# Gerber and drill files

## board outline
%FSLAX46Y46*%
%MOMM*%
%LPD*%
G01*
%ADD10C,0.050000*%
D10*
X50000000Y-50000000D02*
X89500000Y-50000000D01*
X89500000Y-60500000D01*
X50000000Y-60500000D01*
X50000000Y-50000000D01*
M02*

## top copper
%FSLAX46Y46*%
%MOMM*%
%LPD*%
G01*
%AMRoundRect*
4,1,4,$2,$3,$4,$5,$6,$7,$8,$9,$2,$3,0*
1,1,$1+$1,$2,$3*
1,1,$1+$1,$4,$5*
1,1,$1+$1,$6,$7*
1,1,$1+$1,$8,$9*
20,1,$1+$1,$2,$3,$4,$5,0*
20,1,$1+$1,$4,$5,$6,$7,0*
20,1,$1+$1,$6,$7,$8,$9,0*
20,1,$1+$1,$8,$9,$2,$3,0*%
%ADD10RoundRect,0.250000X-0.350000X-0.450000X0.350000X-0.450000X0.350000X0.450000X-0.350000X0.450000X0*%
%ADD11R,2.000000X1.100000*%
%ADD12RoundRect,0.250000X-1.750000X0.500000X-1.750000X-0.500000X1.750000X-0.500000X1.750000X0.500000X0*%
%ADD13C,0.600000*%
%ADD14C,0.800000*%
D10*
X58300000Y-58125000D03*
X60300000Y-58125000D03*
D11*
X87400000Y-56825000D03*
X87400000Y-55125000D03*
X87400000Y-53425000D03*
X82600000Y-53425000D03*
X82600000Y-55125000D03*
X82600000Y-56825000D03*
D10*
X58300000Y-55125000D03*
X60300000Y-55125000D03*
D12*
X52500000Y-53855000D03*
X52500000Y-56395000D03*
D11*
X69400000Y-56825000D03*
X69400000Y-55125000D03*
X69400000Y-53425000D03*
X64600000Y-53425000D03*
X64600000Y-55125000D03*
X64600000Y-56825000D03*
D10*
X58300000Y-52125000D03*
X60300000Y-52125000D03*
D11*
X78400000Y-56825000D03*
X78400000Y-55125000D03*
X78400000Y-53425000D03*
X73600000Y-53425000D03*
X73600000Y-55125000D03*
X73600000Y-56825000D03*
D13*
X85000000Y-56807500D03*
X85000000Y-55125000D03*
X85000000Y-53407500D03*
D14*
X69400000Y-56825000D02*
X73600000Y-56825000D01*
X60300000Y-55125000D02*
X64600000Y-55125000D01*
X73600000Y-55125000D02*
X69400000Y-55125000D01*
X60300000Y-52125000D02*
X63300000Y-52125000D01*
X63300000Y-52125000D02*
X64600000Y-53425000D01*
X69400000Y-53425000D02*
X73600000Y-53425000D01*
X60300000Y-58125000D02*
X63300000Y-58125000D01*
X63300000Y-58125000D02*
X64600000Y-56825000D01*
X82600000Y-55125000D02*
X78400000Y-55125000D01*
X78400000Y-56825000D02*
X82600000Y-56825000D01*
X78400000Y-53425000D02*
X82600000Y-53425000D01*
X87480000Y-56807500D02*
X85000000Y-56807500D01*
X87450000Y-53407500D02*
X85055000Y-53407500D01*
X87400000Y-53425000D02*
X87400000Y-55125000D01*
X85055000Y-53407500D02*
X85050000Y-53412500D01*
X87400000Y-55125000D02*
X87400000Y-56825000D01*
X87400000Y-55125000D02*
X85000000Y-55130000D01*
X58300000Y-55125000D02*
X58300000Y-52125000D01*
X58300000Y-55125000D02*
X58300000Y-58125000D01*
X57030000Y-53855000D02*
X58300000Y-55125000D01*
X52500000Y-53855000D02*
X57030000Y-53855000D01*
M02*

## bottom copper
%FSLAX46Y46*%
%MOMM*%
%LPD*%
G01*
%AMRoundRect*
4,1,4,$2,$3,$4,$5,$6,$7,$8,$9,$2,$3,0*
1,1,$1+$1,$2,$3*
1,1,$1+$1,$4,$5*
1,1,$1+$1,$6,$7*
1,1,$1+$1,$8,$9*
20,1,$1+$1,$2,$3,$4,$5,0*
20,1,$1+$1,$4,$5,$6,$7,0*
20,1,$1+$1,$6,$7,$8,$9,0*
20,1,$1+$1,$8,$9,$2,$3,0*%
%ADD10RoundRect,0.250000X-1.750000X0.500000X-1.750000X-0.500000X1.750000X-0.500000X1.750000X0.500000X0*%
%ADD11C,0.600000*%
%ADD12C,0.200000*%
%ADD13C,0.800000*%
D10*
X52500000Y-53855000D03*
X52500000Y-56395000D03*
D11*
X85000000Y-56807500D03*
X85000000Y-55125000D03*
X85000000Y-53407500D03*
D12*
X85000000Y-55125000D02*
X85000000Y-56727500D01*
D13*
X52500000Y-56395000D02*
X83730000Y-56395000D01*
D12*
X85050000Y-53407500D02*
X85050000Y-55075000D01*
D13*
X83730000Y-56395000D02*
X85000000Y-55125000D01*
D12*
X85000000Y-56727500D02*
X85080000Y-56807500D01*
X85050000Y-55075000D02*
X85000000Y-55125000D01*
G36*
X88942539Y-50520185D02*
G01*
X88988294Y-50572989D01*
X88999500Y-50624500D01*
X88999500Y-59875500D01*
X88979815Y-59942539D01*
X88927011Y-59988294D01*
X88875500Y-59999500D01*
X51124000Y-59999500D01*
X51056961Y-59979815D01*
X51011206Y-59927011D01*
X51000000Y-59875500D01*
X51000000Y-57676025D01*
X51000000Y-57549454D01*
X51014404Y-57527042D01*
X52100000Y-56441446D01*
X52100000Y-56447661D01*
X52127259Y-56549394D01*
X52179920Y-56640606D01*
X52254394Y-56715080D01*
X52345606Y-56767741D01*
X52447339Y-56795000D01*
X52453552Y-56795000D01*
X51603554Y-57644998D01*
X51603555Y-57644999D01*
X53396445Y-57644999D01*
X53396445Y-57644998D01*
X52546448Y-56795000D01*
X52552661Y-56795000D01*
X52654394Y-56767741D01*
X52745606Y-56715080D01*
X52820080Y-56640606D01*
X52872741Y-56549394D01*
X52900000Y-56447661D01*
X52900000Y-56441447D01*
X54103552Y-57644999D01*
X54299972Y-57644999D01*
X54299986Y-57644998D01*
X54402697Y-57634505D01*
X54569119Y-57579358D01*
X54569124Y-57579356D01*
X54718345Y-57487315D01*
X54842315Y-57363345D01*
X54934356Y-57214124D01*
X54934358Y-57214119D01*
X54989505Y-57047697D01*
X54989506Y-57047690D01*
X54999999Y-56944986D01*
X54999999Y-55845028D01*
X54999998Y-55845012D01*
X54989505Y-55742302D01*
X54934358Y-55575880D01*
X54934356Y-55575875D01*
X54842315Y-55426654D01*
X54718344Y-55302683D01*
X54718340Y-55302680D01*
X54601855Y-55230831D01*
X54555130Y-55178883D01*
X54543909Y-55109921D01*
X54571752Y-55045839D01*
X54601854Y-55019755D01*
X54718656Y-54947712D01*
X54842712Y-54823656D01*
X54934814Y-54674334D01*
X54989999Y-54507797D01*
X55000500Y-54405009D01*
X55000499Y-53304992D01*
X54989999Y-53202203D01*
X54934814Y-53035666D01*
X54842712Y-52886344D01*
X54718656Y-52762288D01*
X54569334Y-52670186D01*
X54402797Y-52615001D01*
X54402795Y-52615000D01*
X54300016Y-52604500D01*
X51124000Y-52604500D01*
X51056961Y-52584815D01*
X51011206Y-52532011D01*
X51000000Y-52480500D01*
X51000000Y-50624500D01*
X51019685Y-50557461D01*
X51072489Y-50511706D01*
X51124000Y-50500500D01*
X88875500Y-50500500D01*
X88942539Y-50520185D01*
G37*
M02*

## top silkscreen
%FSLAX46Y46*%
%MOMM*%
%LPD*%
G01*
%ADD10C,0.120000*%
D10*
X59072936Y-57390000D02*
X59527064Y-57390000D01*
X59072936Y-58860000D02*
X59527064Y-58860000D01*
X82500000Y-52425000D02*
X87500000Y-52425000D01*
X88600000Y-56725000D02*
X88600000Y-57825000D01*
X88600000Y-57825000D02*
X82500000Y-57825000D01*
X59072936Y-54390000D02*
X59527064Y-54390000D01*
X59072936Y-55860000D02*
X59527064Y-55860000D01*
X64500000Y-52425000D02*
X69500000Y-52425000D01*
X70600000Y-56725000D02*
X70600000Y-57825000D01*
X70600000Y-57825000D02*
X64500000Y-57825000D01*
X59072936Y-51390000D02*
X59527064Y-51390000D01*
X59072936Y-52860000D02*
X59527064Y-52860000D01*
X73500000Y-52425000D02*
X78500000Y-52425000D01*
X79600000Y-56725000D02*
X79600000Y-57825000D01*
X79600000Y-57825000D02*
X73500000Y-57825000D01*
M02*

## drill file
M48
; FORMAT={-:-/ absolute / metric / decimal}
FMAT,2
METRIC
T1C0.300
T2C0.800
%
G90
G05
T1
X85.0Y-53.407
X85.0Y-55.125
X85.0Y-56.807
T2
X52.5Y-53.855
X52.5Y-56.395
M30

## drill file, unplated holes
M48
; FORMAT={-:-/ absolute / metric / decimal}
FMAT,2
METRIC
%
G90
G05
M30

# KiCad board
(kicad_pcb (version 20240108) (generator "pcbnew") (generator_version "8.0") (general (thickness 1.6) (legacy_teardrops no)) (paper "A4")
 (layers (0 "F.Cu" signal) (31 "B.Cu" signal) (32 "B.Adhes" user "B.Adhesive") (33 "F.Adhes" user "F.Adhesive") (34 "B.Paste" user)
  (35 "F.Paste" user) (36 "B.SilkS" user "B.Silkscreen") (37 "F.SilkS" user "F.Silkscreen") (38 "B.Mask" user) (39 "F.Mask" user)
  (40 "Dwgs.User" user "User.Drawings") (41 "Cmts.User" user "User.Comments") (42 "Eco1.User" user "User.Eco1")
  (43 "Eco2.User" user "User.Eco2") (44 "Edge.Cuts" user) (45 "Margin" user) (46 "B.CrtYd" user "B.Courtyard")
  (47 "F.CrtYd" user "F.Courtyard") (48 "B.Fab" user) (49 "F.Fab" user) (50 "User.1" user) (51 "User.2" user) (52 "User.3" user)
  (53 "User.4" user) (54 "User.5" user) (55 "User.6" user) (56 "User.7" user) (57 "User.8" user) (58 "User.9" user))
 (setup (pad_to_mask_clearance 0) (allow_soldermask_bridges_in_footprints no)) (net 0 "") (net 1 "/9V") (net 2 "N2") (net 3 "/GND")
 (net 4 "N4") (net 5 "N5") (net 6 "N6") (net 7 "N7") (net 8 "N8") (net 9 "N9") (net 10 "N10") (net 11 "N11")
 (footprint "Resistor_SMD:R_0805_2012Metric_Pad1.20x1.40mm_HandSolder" (layer "F.Cu") (at 59.3 58.125)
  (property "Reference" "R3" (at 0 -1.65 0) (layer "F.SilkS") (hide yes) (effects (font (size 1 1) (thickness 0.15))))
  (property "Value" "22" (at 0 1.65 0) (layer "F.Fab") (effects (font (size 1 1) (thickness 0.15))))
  (fp_line (start -0.227064 -0.735) (end 0.227064 -0.735) (stroke (width 0.12) (type solid)) (layer "F.SilkS"))
  (fp_line (start -0.227064 0.735) (end 0.227064 0.735) (stroke (width 0.12) (type solid)) (layer "F.SilkS"))
  (pad "1" smd roundrect (at -1 0) (size 1.2 1.4) (layers "F.Cu" "F.Paste" "F.Mask") (roundrect_rratio 0.208333) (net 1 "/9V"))
  (pad "2" smd roundrect (at 1 0) (size 1.2 1.4) (layers "F.Cu" "F.Paste" "F.Mask") (roundrect_rratio 0.208333) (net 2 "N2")))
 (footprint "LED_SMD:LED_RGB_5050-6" (layer "F.Cu") (at 85 55.125 180)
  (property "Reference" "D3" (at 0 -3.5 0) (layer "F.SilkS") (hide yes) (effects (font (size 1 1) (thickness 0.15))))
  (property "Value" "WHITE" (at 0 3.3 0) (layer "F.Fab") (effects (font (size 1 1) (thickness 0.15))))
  (fp_line (start 2.5 2.7) (end -2.5 2.7) (stroke (width 0.12) (type solid)) (layer "F.SilkS"))
  (fp_line (start -3.6 -1.6) (end -3.6 -2.7) (stroke (width 0.12) (type solid)) (layer "F.SilkS"))
  (fp_line (start -3.6 -2.7) (end 2.5 -2.7) (stroke (width 0.12) (type solid)) (layer "F.SilkS"))
  (pad "1" smd rect (at -2.4 -1.7 270) (size 1.1 2) (layers "F.Cu" "F.Paste" "F.Mask") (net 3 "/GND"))
  (pad "2" smd rect (at -2.4 0 270) (size 1.1 2) (layers "F.Cu" "F.Paste" "F.Mask") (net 3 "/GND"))
  (pad "3" smd rect (at -2.4 1.7 270) (size 1.1 2) (layers "F.Cu" "F.Paste" "F.Mask") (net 3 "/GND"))
  (pad "4" smd rect (at 2.4 1.7 270) (size 1.1 2) (layers "F.Cu" "F.Paste" "F.Mask") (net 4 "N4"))
  (pad "5" smd rect (at 2.4 0 270) (size 1.1 2) (layers "F.Cu" "F.Paste" "F.Mask") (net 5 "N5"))
  (pad "6" smd rect (at 2.4 -1.7 270) (size 1.1 2) (layers "F.Cu" "F.Paste" "F.Mask") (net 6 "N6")))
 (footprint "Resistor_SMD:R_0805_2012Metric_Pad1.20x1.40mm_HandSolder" (layer "F.Cu") (at 59.3 55.125)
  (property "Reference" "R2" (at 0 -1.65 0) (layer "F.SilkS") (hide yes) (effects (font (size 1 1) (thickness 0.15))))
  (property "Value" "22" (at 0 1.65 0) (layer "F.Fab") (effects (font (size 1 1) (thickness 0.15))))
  (fp_line (start -0.227064 -0.735) (end 0.227064 -0.735) (stroke (width 0.12) (type solid)) (layer "F.SilkS"))
  (fp_line (start -0.227064 0.735) (end 0.227064 0.735) (stroke (width 0.12) (type solid)) (layer "F.SilkS"))
  (pad "1" smd roundrect (at -1 0) (size 1.2 1.4) (layers "F.Cu" "F.Paste" "F.Mask") (roundrect_rratio 0.208333) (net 1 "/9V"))
  (pad "2" smd roundrect (at 1 0) (size 1.2 1.4) (layers "F.Cu" "F.Paste" "F.Mask") (roundrect_rratio 0.208333) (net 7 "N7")))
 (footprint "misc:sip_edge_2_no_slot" (layer "F.Cu") (at 50.5 55.125 -90)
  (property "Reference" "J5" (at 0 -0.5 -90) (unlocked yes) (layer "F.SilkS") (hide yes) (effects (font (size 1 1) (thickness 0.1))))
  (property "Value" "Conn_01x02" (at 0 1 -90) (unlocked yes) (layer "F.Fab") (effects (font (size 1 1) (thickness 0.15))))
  (pad "1" thru_hole roundrect (at -1.27 -2 270) (size 1.5 4) (drill 0.8) (layers "*.Cu" "*.Mask") (remove_unused_layers no)
   (roundrect_rratio 0.1666666667) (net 1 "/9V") (thermal_bridge_angle 45))
  (pad "2" thru_hole roundrect (at 1.27 -2 270) (size 1.5 4) (drill 0.8) (layers "*.Cu" "*.Mask") (remove_unused_layers no)
   (roundrect_rratio 0.1666666667) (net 3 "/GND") (thermal_bridge_angle 45)))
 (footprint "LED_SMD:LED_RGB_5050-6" (layer "F.Cu") (at 67 55.125 180)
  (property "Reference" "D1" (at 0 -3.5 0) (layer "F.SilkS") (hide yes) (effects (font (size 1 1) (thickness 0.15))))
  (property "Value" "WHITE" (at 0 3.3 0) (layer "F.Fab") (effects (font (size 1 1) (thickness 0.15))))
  (fp_line (start 2.5 2.7) (end -2.5 2.7) (stroke (width 0.12) (type solid)) (layer "F.SilkS"))
  (fp_line (start -3.6 -1.6) (end -3.6 -2.7) (stroke (width 0.12) (type solid)) (layer "F.SilkS"))
  (fp_line (start -3.6 -2.7) (end 2.5 -2.7) (stroke (width 0.12) (type solid)) (layer "F.SilkS"))
  (pad "1" smd rect (at -2.4 -1.7 270) (size 1.1 2) (layers "F.Cu" "F.Paste" "F.Mask") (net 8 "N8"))
  (pad "2" smd rect (at -2.4 0 270) (size 1.1 2) (layers "F.Cu" "F.Paste" "F.Mask") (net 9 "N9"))
  (pad "3" smd rect (at -2.4 1.7 270) (size 1.1 2) (layers "F.Cu" "F.Paste" "F.Mask") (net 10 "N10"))
  (pad "4" smd rect (at 2.4 1.7 270) (size 1.1 2) (layers "F.Cu" "F.Paste" "F.Mask") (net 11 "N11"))
  (pad "5" smd rect (at 2.4 0 270) (size 1.1 2) (layers "F.Cu" "F.Paste" "F.Mask") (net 7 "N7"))
  (pad "6" smd rect (at 2.4 -1.7 270) (size 1.1 2) (layers "F.Cu" "F.Paste" "F.Mask") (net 2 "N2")))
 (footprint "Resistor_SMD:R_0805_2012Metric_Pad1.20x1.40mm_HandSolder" (layer "F.Cu") (at 59.3 52.125)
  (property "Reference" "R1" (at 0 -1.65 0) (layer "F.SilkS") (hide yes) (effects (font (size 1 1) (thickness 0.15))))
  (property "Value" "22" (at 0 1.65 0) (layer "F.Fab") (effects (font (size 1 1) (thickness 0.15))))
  (fp_line (start -0.227064 -0.735) (end 0.227064 -0.735) (stroke (width 0.12) (type solid)) (layer "F.SilkS"))
  (fp_line (start -0.227064 0.735) (end 0.227064 0.735) (stroke (width 0.12) (type solid)) (layer "F.SilkS"))
  (pad "1" smd roundrect (at -1 0) (size 1.2 1.4) (layers "F.Cu" "F.Paste" "F.Mask") (roundrect_rratio 0.208333) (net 1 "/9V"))
  (pad "2" smd roundrect (at 1 0) (size 1.2 1.4) (layers "F.Cu" "F.Paste" "F.Mask") (roundrect_rratio 0.208333) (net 11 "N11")))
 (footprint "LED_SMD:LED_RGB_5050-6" (layer "F.Cu") (at 76 55.125 180)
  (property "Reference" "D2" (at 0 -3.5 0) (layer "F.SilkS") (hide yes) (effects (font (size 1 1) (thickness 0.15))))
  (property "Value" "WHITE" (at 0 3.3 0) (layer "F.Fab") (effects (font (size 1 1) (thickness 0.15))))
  (fp_line (start 2.5 2.7) (end -2.5 2.7) (stroke (width 0.12) (type solid)) (layer "F.SilkS"))
  (fp_line (start -3.6 -1.6) (end -3.6 -2.7) (stroke (width 0.12) (type solid)) (layer "F.SilkS"))
  (fp_line (start -3.6 -2.7) (end 2.5 -2.7) (stroke (width 0.12) (type solid)) (layer "F.SilkS"))
  (pad "1" smd rect (at -2.4 -1.7 270) (size 1.1 2) (layers "F.Cu" "F.Paste" "F.Mask") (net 6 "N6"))
  (pad "2" smd rect (at -2.4 0 270) (size 1.1 2) (layers "F.Cu" "F.Paste" "F.Mask") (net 5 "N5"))
  (pad "3" smd rect (at -2.4 1.7 270) (size 1.1 2) (layers "F.Cu" "F.Paste" "F.Mask") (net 4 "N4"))
  (pad "4" smd rect (at 2.4 1.7 270) (size 1.1 2) (layers "F.Cu" "F.Paste" "F.Mask") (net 10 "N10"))
  (pad "5" smd rect (at 2.4 0 270) (size 1.1 2) (layers "F.Cu" "F.Paste" "F.Mask") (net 9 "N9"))
  (pad "6" smd rect (at 2.4 -1.7 270) (size 1.1 2) (layers "F.Cu" "F.Paste" "F.Mask") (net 8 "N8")))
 (gr_rect (start 50 50) (end 89.5 60.5) (stroke (width 0.05) (type default)) (fill none) (layer "Edge.Cuts"))
 (segment (start 69.4 56.825) (end 73.6 56.825) (width 0.8) (layer "F.Cu") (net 8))
 (segment (start 60.3 55.125) (end 64.6 55.125) (width 0.8) (layer "F.Cu") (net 7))
 (segment (start 73.6 55.125) (end 69.4 55.125) (width 0.8) (layer "F.Cu") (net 9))
 (segment (start 60.3 52.125) (end 63.3 52.125) (width 0.8) (layer "F.Cu") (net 11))
 (segment (start 63.3 52.125) (end 64.6 53.425) (width 0.8) (layer "F.Cu") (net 11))
 (segment (start 69.4 53.425) (end 73.6 53.425) (width 0.8) (layer "F.Cu") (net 10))
 (segment (start 60.3 58.125) (end 63.3 58.125) (width 0.8) (layer "F.Cu") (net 2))
 (segment (start 63.3 58.125) (end 64.6 56.825) (width 0.8) (layer "F.Cu") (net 2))
 (segment (start 82.6 55.125) (end 78.4 55.125) (width 0.8) (layer "F.Cu") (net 5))
 (segment (start 78.4 56.825) (end 82.6 56.825) (width 0.8) (layer "F.Cu") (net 6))
 (segment (start 78.4 53.425) (end 82.6 53.425) (width 0.8) (layer "F.Cu") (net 4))
 (segment (start 87.48 56.8075) (end 85 56.8075) (width 0.8) (layer "F.Cu") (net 3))
 (segment (start 87.45 53.4075) (end 85.055 53.4075) (width 0.8) (layer "F.Cu") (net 3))
 (segment (start 87.4 53.425) (end 87.4 55.125) (width 0.8) (layer "F.Cu") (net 3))
 (segment (start 85.055 53.4075) (end 85.05 53.4125) (width 0.8) (layer "F.Cu") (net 3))
 (segment (start 87.4 55.125) (end 87.4 56.825) (width 0.8) (layer "F.Cu") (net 3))
 (segment (start 87.4 55.125) (end 85 55.13) (width 0.8) (layer "F.Cu") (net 3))
 (via (at 85 56.8075) (size 0.6) (drill 0.3) (layers "F.Cu" "B.Cu") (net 3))
 (via (at 85 55.125) (size 0.6) (drill 0.3) (layers "F.Cu" "B.Cu") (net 3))
 (via (at 85 53.4075) (size 0.6) (drill 0.3) (layers "F.Cu" "B.Cu") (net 3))
 (segment (start 85 55.125) (end 85 56.7275) (width 0.2) (layer "B.Cu") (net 3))
 (segment (start 52.5 56.395) (end 83.73 56.395) (width 0.8) (layer "B.Cu") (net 3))
 (segment (start 85.05 53.4075) (end 85.05 55.075) (width 0.2) (layer "B.Cu") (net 3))
 (segment (start 83.73 56.395) (end 85 55.125) (width 0.8) (layer "B.Cu") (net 3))
 (segment (start 85 56.7275) (end 85.08 56.8075) (width 0.2) (layer "B.Cu") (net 3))
 (segment (start 85.05 55.075) (end 85 55.125) (width 0.2) (layer "B.Cu") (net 3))
 (segment (start 58.3 55.125) (end 58.3 52.125) (width 0.8) (layer "F.Cu") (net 1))
 (segment (start 58.3 55.125) (end 58.3 58.125) (width 0.8) (layer "F.Cu") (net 1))
 (segment (start 57.03 53.855) (end 58.3 55.125) (width 0.8) (layer "F.Cu") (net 1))
 (segment (start 52.5 53.855) (end 57.03 53.855) (width 0.8) (layer "F.Cu") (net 1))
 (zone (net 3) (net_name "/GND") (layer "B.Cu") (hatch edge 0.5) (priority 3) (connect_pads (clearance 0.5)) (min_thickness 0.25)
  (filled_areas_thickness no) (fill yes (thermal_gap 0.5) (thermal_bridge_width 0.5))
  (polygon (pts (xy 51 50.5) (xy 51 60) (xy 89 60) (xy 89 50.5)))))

